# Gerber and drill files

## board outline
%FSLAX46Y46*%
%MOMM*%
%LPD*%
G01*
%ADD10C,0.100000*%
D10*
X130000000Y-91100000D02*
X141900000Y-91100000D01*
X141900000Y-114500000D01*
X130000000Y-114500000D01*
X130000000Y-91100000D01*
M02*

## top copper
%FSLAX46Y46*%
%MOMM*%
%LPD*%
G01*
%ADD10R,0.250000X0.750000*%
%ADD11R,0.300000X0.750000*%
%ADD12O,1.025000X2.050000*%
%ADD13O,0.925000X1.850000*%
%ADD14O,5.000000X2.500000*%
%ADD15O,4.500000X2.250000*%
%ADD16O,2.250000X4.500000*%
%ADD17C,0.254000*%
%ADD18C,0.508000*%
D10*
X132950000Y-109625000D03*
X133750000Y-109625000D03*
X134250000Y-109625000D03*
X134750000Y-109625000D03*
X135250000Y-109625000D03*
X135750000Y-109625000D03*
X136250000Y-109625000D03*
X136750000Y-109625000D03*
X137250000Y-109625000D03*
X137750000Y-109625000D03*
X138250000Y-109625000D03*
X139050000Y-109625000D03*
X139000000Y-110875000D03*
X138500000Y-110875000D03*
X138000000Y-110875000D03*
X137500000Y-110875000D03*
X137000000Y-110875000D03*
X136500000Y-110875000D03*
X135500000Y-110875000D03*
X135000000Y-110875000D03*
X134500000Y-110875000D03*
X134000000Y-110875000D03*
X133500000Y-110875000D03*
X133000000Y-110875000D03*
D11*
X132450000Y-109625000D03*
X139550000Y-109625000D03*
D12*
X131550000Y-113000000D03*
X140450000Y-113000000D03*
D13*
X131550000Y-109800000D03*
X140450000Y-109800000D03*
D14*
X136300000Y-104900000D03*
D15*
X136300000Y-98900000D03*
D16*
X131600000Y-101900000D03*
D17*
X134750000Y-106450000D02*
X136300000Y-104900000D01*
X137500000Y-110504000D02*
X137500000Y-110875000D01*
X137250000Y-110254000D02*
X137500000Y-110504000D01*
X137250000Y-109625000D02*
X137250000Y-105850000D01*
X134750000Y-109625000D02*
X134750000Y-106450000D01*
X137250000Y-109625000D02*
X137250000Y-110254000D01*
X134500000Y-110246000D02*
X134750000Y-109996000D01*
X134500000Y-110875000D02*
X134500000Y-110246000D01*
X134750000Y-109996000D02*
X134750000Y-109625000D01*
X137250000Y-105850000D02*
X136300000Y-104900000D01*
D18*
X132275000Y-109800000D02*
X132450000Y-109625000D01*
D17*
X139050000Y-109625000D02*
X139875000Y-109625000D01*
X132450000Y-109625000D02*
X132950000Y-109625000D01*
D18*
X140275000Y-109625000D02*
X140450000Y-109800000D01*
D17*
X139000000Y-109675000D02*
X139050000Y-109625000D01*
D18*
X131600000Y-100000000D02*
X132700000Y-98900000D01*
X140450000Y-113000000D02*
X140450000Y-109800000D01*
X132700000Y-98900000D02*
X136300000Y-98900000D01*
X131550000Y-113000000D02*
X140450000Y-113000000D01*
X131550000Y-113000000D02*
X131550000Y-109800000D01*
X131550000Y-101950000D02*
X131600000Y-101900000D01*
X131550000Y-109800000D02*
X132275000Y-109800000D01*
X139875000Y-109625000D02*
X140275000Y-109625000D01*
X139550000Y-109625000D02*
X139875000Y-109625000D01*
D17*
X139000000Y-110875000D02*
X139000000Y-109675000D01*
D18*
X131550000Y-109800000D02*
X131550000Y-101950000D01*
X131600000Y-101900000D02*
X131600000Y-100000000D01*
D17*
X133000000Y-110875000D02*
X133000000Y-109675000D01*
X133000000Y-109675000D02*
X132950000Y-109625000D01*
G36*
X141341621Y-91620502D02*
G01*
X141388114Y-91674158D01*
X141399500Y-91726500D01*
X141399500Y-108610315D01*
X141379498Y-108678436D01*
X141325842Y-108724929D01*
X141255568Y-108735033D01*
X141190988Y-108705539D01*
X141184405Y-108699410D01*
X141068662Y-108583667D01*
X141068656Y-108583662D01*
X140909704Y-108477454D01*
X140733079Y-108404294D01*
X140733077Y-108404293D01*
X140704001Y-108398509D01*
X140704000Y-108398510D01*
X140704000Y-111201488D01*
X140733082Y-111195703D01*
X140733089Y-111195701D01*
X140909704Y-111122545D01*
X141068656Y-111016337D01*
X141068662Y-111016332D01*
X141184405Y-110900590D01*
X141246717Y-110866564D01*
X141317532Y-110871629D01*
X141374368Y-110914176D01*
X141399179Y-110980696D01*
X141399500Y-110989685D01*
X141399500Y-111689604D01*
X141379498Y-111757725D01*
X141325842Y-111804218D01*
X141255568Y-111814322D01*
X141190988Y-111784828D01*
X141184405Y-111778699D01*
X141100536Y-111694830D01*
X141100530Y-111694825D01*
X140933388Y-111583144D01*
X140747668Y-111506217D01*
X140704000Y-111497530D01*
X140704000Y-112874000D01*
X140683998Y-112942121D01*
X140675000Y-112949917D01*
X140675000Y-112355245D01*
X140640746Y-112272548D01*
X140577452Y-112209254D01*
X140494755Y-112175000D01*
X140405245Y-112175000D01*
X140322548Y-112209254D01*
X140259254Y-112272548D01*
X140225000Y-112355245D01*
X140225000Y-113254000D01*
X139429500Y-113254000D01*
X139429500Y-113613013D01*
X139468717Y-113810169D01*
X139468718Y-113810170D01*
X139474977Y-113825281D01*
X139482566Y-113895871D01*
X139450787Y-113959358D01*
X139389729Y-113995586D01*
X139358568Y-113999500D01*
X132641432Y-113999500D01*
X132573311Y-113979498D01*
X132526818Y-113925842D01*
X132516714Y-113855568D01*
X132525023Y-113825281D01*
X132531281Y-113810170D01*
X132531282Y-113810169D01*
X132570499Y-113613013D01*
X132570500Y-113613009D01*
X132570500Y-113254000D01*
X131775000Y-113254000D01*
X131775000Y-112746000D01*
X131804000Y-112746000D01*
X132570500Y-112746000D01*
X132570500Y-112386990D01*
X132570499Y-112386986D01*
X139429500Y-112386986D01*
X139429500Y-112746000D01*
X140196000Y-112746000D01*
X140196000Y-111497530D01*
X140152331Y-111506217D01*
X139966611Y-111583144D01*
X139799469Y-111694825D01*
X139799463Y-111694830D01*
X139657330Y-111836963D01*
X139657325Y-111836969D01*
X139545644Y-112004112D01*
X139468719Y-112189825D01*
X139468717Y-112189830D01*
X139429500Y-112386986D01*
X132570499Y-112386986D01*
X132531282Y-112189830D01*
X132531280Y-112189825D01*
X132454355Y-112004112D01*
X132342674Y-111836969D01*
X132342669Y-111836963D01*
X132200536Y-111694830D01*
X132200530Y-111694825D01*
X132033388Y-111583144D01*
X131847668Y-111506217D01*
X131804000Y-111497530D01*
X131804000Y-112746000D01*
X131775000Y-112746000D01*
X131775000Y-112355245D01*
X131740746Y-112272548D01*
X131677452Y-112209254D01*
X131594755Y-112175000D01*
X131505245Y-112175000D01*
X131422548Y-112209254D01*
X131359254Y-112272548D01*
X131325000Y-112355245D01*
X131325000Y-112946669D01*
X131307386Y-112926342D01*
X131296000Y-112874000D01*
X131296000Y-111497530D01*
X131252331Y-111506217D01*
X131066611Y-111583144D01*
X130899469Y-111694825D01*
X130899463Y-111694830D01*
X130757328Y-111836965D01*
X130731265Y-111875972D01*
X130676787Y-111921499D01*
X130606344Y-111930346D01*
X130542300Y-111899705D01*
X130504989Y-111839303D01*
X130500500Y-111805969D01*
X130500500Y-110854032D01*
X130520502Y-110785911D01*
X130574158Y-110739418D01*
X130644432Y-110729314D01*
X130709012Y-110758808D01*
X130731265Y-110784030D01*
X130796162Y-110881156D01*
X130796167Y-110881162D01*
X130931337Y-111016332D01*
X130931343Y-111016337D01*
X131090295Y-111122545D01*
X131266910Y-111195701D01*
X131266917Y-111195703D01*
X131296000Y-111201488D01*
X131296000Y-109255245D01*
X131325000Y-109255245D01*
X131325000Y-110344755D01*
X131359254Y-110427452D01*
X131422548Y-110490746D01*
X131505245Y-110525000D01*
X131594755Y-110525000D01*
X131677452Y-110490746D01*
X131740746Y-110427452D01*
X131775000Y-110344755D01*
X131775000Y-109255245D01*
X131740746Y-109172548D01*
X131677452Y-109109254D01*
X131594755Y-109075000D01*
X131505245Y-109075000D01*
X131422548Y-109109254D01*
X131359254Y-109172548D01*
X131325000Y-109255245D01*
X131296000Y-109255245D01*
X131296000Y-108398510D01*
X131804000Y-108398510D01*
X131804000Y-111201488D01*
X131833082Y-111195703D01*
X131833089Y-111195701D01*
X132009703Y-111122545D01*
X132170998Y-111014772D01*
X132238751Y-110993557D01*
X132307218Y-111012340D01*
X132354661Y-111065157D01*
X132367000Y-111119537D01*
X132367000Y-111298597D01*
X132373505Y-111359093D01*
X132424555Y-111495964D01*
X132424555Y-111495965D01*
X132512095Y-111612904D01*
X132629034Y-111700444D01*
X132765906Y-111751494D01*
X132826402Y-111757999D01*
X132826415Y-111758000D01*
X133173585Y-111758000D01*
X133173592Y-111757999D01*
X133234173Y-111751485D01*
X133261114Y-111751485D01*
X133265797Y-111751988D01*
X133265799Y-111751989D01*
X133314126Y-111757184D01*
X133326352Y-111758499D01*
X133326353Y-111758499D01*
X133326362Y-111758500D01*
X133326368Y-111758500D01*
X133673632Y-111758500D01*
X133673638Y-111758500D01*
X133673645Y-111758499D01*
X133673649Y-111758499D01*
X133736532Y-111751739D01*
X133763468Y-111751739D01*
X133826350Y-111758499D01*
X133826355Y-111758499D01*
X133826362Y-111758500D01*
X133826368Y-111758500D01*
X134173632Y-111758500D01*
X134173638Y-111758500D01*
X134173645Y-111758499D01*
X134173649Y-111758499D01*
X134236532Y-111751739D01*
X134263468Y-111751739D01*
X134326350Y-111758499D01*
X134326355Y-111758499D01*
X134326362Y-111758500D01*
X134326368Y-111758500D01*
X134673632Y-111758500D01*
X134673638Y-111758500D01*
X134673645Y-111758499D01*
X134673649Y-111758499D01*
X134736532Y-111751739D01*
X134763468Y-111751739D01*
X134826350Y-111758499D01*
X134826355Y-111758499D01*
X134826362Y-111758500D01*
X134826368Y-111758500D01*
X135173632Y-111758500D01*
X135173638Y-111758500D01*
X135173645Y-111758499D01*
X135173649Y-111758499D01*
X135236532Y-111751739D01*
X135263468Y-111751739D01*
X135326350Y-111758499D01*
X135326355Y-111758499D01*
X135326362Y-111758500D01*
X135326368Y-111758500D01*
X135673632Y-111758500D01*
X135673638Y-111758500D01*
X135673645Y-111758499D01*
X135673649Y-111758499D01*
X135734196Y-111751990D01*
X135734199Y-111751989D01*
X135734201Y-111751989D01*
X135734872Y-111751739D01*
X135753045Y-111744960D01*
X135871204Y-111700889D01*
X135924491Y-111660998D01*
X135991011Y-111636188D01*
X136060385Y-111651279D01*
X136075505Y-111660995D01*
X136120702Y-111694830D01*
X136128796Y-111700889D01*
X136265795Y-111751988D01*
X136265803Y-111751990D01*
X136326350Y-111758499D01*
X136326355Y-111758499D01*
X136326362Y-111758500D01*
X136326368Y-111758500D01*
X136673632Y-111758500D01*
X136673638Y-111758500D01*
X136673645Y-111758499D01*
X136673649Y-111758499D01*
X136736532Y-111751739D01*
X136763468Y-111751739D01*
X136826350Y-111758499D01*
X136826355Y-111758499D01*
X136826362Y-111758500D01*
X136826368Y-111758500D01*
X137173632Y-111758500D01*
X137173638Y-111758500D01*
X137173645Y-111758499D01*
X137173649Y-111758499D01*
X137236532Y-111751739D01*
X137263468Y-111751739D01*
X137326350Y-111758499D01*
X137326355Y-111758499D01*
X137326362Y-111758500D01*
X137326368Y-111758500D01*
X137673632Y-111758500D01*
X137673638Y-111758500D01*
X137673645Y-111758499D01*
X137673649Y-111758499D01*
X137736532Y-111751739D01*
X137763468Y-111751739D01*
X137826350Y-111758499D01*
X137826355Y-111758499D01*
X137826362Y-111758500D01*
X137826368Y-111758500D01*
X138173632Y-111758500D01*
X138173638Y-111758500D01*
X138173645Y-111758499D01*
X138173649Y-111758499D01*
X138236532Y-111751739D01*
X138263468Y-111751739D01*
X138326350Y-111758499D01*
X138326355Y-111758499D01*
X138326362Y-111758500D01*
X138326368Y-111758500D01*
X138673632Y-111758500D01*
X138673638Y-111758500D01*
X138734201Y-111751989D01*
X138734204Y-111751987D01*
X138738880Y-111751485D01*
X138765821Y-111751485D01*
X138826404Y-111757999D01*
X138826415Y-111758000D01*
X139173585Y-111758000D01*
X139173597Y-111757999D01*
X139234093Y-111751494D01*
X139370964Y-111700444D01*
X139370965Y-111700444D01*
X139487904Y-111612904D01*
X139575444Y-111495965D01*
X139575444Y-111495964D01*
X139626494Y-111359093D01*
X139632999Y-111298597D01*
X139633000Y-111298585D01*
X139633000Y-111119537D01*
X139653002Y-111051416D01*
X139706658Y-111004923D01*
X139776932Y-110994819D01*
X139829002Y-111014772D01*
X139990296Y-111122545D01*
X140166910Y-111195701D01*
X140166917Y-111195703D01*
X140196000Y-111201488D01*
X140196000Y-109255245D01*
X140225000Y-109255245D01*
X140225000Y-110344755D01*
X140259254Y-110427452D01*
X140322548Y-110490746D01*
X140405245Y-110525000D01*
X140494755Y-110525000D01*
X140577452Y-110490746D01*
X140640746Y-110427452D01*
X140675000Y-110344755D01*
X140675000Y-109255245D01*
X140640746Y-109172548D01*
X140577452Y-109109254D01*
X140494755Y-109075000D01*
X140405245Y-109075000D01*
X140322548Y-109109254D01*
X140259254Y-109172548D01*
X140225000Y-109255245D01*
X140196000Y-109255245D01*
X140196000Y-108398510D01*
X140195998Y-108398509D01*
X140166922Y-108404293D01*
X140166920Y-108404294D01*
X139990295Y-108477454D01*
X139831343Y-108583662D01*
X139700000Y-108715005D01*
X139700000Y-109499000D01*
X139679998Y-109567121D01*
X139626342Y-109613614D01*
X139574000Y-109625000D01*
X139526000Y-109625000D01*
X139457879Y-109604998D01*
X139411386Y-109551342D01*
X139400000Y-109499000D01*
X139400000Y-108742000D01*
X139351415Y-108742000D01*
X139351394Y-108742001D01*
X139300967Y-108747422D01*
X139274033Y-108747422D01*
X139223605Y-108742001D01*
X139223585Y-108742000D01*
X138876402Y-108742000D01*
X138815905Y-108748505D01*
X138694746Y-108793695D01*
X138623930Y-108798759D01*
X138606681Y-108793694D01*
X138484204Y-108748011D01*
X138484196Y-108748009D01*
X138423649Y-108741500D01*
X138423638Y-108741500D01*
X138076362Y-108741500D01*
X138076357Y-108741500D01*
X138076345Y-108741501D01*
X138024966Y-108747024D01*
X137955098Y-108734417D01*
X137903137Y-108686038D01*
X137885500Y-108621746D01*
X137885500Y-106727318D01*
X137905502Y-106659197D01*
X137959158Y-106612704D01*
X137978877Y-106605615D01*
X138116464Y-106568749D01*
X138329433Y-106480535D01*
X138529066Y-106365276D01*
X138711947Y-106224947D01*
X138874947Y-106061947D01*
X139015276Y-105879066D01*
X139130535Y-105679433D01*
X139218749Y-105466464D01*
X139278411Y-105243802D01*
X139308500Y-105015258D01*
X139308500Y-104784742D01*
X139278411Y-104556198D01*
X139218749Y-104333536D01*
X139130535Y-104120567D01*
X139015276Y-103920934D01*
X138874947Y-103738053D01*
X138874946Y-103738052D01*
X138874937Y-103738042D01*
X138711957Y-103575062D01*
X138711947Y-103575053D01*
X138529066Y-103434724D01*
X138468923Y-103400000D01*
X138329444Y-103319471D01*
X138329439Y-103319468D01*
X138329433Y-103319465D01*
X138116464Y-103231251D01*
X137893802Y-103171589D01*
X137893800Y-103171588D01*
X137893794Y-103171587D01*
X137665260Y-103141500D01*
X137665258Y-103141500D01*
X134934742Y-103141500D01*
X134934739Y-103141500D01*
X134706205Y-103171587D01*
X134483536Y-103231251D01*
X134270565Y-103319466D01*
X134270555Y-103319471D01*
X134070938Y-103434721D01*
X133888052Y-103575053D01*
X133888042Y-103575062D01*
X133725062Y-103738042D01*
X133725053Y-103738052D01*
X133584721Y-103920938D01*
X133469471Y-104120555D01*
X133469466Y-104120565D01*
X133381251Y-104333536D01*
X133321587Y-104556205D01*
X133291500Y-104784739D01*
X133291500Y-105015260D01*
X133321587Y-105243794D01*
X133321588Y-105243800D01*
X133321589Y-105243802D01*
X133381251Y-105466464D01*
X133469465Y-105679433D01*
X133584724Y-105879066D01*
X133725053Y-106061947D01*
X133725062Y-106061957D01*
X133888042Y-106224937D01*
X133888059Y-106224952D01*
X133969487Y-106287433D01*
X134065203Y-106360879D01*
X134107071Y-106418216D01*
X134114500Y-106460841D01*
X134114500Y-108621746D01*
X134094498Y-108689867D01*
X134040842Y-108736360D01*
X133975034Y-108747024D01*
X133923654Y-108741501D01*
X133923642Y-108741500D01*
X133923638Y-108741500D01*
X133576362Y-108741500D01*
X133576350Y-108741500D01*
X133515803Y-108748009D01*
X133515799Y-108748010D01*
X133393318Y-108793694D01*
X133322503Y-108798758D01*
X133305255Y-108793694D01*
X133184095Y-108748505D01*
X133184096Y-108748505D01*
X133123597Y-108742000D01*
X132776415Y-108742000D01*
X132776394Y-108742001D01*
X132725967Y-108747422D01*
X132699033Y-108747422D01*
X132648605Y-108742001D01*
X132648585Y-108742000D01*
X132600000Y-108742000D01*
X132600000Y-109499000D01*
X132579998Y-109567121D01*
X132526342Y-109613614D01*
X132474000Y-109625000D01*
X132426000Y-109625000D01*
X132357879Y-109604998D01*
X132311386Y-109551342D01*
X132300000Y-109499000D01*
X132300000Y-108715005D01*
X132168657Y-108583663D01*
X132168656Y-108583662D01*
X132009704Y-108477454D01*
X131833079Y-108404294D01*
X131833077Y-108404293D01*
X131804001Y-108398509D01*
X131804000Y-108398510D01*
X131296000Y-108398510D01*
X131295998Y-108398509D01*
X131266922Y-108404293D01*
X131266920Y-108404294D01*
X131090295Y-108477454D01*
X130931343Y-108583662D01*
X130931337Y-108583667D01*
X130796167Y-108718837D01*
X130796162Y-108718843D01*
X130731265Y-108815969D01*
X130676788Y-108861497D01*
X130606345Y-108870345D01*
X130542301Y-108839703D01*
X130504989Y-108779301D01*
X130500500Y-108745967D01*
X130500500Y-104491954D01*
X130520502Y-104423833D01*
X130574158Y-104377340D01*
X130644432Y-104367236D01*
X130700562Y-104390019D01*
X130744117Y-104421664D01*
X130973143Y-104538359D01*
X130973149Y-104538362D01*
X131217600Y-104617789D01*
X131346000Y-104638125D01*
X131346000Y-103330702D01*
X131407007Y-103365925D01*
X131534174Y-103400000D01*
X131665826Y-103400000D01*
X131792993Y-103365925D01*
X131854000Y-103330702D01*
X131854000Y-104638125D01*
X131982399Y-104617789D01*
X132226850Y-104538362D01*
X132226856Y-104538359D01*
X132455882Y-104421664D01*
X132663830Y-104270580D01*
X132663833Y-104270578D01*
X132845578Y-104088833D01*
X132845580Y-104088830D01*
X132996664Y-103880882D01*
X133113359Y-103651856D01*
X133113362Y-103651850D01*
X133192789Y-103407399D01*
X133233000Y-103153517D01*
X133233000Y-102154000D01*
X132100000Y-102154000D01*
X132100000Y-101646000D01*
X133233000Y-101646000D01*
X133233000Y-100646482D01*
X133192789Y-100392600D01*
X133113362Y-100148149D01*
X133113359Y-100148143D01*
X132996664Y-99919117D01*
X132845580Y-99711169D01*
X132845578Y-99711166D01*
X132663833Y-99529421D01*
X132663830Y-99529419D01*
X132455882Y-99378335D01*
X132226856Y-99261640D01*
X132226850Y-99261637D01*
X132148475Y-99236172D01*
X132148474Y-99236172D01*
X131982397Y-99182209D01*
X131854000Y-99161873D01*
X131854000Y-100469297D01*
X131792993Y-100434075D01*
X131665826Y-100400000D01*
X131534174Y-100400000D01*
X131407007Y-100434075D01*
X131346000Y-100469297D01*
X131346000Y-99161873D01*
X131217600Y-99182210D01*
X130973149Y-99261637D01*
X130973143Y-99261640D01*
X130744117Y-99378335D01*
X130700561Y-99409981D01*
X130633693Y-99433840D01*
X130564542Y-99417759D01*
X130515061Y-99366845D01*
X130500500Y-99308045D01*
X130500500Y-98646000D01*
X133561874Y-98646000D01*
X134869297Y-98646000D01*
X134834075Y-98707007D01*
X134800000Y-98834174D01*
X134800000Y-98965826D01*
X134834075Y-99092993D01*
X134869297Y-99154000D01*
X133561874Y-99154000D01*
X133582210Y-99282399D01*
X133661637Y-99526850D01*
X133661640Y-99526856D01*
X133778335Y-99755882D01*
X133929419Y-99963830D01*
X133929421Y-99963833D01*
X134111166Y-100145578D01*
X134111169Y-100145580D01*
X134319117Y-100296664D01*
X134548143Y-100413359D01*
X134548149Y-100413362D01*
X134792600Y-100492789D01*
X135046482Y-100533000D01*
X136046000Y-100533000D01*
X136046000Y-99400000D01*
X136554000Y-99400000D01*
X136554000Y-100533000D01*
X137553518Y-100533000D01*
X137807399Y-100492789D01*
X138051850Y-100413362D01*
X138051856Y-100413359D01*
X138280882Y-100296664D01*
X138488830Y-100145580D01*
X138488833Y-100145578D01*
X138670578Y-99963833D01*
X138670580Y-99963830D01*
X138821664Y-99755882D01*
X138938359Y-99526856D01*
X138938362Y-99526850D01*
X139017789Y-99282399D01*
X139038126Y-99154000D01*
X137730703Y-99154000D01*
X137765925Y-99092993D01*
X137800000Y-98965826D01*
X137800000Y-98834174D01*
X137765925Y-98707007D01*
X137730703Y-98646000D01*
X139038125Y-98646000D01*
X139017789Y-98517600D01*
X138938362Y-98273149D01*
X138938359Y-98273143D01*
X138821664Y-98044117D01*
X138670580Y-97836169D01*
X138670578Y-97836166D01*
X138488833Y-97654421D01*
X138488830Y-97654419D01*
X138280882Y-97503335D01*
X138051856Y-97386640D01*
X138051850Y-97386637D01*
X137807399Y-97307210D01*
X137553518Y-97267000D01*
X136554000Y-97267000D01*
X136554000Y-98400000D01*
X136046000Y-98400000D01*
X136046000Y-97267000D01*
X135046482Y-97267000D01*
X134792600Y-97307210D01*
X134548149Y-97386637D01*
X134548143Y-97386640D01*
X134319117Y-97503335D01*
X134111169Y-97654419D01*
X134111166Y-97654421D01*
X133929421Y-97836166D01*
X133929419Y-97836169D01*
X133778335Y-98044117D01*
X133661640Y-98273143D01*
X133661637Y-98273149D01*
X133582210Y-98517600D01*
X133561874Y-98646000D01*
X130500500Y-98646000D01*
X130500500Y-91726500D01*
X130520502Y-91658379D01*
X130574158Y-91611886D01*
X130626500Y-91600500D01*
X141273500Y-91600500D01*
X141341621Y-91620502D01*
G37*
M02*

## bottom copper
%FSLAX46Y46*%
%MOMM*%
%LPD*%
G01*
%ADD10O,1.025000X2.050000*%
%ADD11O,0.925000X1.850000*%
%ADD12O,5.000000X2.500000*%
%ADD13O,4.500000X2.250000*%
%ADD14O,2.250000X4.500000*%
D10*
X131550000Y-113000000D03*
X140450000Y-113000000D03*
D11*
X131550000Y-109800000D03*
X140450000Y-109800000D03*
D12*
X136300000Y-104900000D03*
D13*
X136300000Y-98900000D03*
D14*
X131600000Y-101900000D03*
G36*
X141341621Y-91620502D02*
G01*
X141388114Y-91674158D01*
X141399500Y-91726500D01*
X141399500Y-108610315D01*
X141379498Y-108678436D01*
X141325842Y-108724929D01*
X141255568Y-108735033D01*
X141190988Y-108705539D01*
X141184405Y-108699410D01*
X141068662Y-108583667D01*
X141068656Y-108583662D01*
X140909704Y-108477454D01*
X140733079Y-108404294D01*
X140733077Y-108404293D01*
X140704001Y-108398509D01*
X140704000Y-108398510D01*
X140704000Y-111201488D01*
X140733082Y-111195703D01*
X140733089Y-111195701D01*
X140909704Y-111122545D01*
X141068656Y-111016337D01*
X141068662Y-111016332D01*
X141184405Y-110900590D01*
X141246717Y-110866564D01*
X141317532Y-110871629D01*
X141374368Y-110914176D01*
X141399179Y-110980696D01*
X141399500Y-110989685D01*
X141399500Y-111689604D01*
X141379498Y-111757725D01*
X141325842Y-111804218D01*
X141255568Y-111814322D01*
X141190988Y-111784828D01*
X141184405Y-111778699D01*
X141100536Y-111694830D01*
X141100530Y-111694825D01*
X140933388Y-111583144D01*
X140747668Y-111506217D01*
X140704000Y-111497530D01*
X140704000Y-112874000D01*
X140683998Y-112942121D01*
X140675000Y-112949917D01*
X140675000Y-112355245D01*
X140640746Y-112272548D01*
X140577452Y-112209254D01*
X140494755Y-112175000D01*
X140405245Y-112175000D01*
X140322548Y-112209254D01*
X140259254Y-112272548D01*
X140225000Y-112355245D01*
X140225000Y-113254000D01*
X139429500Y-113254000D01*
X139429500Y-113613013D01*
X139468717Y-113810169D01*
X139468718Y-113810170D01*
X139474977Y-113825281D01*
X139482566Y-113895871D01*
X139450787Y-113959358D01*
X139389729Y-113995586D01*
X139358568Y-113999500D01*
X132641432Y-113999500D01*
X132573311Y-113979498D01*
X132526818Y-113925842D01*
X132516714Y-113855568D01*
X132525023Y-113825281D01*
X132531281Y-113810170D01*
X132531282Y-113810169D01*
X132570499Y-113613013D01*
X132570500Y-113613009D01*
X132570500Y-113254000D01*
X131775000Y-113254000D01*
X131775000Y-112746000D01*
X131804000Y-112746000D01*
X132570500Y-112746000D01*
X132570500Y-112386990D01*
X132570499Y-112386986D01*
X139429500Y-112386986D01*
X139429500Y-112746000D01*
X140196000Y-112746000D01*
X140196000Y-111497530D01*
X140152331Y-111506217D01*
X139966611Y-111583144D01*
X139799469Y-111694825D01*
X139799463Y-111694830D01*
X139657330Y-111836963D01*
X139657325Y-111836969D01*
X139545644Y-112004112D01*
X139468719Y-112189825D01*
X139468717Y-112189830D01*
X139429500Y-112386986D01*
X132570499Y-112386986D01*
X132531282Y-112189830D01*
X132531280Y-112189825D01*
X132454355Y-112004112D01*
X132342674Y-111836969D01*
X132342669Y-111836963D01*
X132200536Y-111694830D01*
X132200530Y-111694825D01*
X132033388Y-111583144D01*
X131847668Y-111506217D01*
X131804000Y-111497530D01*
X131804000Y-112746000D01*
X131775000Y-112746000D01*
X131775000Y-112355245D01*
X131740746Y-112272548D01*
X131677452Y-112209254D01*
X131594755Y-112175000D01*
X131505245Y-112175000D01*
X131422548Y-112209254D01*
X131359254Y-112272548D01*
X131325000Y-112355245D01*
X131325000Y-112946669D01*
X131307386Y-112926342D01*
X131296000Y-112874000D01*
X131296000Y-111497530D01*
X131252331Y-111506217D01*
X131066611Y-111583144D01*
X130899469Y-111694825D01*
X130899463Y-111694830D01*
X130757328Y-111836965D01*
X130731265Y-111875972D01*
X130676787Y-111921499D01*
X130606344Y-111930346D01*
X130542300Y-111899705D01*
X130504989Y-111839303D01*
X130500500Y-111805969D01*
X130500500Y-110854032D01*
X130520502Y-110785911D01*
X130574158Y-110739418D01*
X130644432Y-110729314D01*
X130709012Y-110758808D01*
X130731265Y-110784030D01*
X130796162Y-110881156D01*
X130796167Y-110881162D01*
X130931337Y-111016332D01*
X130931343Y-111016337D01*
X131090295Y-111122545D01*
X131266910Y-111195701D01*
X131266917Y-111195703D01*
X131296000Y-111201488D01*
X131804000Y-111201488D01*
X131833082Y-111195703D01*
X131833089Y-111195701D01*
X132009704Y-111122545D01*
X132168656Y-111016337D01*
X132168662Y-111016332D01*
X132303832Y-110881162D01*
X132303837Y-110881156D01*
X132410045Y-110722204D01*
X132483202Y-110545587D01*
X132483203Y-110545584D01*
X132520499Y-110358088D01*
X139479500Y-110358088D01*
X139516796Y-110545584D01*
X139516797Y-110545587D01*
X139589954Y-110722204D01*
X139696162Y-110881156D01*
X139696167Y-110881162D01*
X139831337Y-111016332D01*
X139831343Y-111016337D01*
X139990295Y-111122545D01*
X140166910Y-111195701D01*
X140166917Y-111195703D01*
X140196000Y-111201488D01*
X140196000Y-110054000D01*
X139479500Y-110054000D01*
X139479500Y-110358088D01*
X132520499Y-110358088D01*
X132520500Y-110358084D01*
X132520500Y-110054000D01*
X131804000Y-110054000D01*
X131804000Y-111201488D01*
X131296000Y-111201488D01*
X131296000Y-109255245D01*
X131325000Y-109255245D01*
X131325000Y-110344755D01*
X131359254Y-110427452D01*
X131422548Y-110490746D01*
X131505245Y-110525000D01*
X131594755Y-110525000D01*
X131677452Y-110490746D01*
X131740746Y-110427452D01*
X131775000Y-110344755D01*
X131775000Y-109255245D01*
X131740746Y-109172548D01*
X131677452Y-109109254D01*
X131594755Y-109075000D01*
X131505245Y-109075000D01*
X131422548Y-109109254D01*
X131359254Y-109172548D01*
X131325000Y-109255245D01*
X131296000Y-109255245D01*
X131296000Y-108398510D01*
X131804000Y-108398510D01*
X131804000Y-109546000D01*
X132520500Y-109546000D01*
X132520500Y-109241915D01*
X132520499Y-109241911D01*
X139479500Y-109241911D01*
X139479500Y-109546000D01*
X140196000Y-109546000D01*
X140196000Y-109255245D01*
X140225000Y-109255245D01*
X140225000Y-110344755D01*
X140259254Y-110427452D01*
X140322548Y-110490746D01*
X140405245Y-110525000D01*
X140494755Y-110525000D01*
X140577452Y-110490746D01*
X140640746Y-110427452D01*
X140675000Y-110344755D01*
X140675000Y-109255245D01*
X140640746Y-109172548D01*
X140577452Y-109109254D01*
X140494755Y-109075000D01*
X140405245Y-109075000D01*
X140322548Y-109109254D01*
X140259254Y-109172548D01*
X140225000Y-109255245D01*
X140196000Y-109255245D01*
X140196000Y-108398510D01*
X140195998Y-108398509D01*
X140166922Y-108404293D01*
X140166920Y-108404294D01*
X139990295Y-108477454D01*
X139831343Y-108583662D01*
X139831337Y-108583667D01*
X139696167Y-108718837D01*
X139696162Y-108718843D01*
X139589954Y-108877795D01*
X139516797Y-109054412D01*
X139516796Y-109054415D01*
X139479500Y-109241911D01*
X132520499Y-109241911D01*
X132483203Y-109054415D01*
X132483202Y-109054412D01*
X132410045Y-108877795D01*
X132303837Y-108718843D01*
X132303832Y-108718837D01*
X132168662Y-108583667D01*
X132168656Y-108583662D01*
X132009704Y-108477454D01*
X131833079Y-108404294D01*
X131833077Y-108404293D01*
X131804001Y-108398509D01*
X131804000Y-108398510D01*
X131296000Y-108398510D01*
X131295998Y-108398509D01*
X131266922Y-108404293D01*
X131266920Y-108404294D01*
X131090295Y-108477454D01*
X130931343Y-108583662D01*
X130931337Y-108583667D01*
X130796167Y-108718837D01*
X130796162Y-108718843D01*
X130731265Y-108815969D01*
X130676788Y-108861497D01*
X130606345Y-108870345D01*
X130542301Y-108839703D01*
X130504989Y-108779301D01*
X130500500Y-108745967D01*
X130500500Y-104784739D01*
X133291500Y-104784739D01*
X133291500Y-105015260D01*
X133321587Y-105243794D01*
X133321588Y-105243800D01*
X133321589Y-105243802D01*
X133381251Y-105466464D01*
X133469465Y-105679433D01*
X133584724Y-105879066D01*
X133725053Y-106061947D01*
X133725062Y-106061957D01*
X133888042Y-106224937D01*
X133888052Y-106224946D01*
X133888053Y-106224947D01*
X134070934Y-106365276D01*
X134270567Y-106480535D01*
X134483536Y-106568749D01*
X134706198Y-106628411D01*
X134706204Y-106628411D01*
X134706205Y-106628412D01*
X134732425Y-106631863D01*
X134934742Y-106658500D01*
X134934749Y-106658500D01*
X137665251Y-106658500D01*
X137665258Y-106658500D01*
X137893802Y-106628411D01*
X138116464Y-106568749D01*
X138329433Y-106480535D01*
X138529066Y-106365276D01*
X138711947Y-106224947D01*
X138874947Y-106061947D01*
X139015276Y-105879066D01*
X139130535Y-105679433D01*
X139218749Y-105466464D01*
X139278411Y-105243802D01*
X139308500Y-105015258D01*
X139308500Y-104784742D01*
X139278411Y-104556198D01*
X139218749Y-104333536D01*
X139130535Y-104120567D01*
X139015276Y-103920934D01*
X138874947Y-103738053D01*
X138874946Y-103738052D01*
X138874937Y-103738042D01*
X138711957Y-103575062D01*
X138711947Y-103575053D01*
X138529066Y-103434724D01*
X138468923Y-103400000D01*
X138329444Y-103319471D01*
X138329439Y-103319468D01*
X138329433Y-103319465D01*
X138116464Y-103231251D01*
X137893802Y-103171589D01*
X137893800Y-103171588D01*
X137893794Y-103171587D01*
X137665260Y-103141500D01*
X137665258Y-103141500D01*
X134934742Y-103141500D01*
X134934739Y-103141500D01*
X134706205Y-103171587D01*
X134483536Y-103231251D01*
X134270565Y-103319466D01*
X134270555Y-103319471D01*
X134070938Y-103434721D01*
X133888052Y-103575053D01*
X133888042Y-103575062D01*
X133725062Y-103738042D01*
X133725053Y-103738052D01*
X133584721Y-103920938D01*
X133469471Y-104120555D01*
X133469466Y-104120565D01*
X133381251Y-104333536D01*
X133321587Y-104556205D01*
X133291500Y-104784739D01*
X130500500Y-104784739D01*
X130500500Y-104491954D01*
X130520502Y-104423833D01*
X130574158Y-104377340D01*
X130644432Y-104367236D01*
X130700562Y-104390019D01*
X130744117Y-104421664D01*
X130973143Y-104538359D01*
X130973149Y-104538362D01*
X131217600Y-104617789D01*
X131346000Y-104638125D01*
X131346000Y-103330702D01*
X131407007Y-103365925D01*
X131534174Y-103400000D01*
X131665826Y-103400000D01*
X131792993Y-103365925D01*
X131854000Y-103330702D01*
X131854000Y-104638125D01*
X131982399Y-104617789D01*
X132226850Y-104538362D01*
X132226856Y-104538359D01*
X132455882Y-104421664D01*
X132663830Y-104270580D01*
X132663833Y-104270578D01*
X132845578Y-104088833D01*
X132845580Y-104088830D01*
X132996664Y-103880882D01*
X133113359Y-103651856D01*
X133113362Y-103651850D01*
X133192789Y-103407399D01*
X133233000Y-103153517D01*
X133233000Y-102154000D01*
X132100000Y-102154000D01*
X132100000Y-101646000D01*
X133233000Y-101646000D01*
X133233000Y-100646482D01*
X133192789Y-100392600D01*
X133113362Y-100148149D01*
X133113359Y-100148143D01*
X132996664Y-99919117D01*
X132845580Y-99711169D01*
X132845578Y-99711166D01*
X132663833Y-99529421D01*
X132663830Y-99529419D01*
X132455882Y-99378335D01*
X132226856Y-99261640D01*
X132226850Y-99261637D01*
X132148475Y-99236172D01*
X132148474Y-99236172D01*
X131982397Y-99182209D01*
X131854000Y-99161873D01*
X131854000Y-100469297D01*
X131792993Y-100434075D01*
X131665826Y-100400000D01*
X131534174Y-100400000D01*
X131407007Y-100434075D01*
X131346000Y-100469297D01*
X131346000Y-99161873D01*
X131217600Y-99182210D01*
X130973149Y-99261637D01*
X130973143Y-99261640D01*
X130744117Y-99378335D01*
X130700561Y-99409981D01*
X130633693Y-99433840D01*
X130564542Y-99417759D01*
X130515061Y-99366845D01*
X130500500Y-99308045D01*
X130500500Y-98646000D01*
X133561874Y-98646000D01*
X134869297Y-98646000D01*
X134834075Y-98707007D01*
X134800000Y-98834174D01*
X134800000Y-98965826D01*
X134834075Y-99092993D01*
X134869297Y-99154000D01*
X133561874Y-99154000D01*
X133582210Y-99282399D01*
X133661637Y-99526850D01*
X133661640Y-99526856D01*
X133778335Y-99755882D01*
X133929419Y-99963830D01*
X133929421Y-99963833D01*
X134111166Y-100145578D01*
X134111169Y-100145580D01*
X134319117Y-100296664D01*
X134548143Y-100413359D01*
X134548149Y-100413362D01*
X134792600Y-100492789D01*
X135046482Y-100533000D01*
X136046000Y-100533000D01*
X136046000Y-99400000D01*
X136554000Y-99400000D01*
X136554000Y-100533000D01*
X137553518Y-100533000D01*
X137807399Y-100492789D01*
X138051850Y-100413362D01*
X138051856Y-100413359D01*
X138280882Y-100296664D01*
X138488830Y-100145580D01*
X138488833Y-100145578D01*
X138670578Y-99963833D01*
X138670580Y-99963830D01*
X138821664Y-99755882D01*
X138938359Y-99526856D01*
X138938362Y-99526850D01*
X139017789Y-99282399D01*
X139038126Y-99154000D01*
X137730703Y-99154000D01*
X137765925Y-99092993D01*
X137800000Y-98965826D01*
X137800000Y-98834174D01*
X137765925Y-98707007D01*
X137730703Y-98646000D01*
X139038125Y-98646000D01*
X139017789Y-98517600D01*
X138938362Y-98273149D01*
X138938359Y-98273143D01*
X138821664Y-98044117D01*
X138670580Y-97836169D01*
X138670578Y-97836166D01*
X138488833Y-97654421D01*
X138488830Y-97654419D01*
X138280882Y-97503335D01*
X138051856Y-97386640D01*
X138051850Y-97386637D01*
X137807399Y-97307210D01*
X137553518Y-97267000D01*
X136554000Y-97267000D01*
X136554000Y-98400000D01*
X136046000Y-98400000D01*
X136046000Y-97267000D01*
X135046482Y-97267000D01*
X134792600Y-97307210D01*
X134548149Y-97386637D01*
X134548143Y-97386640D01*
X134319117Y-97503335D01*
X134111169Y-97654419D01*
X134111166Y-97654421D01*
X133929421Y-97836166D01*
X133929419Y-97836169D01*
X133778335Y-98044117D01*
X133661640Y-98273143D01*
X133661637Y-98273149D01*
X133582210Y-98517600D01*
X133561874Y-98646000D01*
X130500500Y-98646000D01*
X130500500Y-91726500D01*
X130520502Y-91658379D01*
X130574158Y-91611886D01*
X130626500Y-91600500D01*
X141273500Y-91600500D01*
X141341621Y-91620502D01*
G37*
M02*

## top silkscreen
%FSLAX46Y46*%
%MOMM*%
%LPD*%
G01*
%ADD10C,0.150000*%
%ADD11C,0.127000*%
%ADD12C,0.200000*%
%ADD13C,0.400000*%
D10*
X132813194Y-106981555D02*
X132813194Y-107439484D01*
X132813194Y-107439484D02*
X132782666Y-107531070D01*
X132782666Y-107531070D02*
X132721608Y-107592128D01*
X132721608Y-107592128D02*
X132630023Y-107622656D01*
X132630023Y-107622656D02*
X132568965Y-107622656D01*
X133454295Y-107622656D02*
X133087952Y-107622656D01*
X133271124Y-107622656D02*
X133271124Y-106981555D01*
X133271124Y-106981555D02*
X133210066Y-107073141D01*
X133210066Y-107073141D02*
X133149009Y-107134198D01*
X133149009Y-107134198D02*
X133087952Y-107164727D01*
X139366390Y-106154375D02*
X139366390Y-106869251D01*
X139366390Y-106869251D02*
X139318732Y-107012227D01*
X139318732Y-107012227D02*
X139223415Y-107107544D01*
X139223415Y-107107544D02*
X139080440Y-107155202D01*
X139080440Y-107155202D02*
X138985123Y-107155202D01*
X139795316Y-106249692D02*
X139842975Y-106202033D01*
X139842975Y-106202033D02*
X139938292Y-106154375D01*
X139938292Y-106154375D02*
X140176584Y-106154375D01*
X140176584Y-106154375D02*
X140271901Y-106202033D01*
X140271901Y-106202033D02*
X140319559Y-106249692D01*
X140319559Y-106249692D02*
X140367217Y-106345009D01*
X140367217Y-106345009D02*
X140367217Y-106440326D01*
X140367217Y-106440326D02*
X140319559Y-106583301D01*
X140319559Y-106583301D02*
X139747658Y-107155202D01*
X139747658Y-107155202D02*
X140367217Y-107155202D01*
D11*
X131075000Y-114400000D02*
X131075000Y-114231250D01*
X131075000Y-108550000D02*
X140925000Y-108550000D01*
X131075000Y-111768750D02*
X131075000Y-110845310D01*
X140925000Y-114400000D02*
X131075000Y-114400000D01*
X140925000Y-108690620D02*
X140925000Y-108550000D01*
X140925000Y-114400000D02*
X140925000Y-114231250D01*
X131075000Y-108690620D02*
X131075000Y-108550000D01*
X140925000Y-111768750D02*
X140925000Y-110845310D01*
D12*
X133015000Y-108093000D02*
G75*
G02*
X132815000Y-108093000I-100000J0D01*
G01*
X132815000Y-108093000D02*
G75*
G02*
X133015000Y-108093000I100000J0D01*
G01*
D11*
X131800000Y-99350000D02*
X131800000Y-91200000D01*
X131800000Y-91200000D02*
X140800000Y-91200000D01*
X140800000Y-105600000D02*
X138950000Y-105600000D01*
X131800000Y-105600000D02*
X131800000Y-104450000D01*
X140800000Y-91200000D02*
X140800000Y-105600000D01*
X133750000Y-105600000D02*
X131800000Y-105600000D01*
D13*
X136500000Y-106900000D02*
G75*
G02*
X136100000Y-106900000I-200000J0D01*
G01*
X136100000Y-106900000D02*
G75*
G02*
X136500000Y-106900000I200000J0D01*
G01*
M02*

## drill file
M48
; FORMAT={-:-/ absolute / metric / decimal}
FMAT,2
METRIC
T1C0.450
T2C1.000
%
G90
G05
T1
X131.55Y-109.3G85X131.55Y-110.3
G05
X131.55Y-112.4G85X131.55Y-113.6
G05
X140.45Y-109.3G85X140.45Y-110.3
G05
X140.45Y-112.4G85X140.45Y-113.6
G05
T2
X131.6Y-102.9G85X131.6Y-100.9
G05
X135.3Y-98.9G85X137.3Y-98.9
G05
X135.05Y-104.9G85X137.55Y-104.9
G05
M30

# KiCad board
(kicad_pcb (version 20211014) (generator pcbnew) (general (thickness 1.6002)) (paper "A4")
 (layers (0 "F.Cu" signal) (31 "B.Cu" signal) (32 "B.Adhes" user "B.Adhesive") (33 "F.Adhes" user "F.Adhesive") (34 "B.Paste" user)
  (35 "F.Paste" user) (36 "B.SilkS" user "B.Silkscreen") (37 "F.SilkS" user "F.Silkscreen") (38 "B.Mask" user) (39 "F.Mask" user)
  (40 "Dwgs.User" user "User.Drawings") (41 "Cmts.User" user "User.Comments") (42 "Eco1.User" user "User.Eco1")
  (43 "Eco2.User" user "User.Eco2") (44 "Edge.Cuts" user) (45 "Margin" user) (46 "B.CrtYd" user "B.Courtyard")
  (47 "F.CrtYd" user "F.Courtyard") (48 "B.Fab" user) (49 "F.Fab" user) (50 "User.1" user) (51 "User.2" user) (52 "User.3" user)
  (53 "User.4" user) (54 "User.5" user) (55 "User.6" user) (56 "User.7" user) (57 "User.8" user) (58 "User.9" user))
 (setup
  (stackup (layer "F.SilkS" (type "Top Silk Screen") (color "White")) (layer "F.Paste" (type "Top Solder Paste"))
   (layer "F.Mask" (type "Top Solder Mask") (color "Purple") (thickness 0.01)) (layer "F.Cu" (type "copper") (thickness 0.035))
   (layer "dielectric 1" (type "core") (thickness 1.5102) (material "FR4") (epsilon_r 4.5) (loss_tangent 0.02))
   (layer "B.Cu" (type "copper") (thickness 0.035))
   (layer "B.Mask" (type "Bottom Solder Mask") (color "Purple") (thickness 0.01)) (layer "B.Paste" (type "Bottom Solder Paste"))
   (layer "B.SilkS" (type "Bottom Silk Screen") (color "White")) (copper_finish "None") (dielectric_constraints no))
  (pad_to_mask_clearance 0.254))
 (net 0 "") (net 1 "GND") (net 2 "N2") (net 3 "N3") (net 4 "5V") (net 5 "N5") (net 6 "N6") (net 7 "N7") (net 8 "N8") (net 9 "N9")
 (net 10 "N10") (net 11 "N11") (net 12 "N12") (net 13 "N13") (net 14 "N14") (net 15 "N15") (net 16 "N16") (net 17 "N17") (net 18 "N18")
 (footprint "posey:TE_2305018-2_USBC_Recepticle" (layer "F.Cu") (at 136 113)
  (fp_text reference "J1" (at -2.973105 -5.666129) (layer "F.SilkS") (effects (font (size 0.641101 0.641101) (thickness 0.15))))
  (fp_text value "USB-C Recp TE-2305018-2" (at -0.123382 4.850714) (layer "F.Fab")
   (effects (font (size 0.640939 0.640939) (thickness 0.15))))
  (fp_line (start -4.925 1.4) (end -4.925 1.23125) (layer "F.SilkS") (width 0.127))
  (fp_line (start -4.925 -4.45) (end 4.925 -4.45) (layer "F.SilkS") (width 0.127))
  (fp_line (start -4.925 -1.23125) (end -4.925 -2.15469) (layer "F.SilkS") (width 0.127))
  (fp_line (start 4.925 1.4) (end -4.925 1.4) (layer "F.SilkS") (width 0.127))
  (fp_line (start 4.925 -4.30938) (end 4.925 -4.45) (layer "F.SilkS") (width 0.127))
  (fp_line (start 4.925 1.4) (end 4.925 1.23125) (layer "F.SilkS") (width 0.127))
  (fp_line (start -4.925 -4.30938) (end -4.925 -4.45) (layer "F.SilkS") (width 0.127))
  (fp_line (start 4.925 -1.23125) (end 4.925 -2.15469) (layer "F.SilkS") (width 0.127))
  (fp_circle (center -3.085 -4.907) (end -2.985 -4.907) (layer "F.SilkS") (width 0.2) (fill none))
  (pad "A1" smd rect (at -3.05 -3.375) (size 0.25 0.75) (layers "F.Cu" "F.Paste" "F.Mask") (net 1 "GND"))
  (pad "A2" smd rect (at -2.25 -3.375) (size 0.25 0.75) (layers "F.Cu" "F.Paste" "F.Mask") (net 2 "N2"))
  (pad "A3" smd rect (at -1.75 -3.375) (size 0.25 0.75) (layers "F.Cu" "F.Paste" "F.Mask") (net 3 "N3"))
  (pad "A4" smd rect (at -1.25 -3.375) (size 0.25 0.75) (layers "F.Cu" "F.Paste" "F.Mask") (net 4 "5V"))
  (pad "A5" smd rect (at -0.75 -3.375) (size 0.25 0.75) (layers "F.Cu" "F.Paste" "F.Mask") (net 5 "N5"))
  (pad "A6" smd rect (at -0.25 -3.375) (size 0.25 0.75) (layers "F.Cu" "F.Paste" "F.Mask") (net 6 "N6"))
  (pad "A7" smd rect (at 0.25 -3.375) (size 0.25 0.75) (layers "F.Cu" "F.Paste" "F.Mask") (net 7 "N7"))
  (pad "A8" smd rect (at 0.75 -3.375) (size 0.25 0.75) (layers "F.Cu" "F.Paste" "F.Mask") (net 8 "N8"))
  (pad "A9" smd rect (at 1.25 -3.375) (size 0.25 0.75) (layers "F.Cu" "F.Paste" "F.Mask") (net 4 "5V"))
  (pad "A10" smd rect (at 1.75 -3.375) (size 0.25 0.75) (layers "F.Cu" "F.Paste" "F.Mask") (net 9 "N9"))
  (pad "A11" smd rect (at 2.25 -3.375) (size 0.25 0.75) (layers "F.Cu" "F.Paste" "F.Mask") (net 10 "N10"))
  (pad "A12" smd rect (at 3.05 -3.375) (size 0.25 0.75) (layers "F.Cu" "F.Paste" "F.Mask") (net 1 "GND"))
  (pad "B1" smd rect (at 3 -2.125) (size 0.25 0.75) (layers "F.Cu" "F.Paste" "F.Mask") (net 1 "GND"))
  (pad "B2" smd rect (at 2.5 -2.125) (size 0.25 0.75) (layers "F.Cu" "F.Paste" "F.Mask") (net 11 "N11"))
  (pad "B3" smd rect (at 2 -2.125) (size 0.25 0.75) (layers "F.Cu" "F.Paste" "F.Mask") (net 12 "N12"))
  (pad "B4" smd rect (at 1.5 -2.125) (size 0.25 0.75) (layers "F.Cu" "F.Paste" "F.Mask") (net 4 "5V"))
  (pad "B5" smd rect (at 1 -2.125) (size 0.25 0.75) (layers "F.Cu" "F.Paste" "F.Mask") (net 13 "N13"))
  (pad "B6" smd rect (at 0.5 -2.125) (size 0.25 0.75) (layers "F.Cu" "F.Paste" "F.Mask") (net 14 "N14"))
  (pad "B7" smd rect (at -0.5 -2.125) (size 0.25 0.75) (layers "F.Cu" "F.Paste" "F.Mask") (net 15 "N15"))
  (pad "B8" smd rect (at -1 -2.125) (size 0.25 0.75) (layers "F.Cu" "F.Paste" "F.Mask") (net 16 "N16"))
  (pad "B9" smd rect (at -1.5 -2.125) (size 0.25 0.75) (layers "F.Cu" "F.Paste" "F.Mask") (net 4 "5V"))
  (pad "B10" smd rect (at -2 -2.125) (size 0.25 0.75) (layers "F.Cu" "F.Paste" "F.Mask") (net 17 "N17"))
  (pad "B11" smd rect (at -2.5 -2.125) (size 0.25 0.75) (layers "F.Cu" "F.Paste" "F.Mask") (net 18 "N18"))
  (pad "B12" smd rect (at -3 -2.125) (size 0.25 0.75) (layers "F.Cu" "F.Paste" "F.Mask") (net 1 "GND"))
  (pad "G1" smd rect (at -3.55 -3.375) (size 0.3 0.75) (layers "F.Cu" "F.Paste" "F.Mask") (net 1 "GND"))
  (pad "G2" smd rect (at 3.55 -3.375) (size 0.3 0.75) (layers "F.Cu" "F.Paste" "F.Mask") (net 1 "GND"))
  (pad "S1" thru_hole oval (at -4.45 0) (size 1.025 2.05) (drill oval 0.45 1.65) (layers *.Cu *.Mask) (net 1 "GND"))
  (pad "S2" thru_hole oval (at 4.45 0) (size 1.025 2.05) (drill oval 0.45 1.65) (layers *.Cu *.Mask) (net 1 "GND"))
  (pad "S3" thru_hole oval (at -4.45 -3.2) (size 0.925 1.85) (drill oval 0.45 1.45) (layers *.Cu *.Mask) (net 1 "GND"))
  (pad "S4" thru_hole oval (at 4.45 -3.2) (size 0.925 1.85) (drill oval 0.45 1.45) (layers *.Cu *.Mask) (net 1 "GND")))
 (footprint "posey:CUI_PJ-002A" (layer "F.Cu") (at 136.3 104.9 90)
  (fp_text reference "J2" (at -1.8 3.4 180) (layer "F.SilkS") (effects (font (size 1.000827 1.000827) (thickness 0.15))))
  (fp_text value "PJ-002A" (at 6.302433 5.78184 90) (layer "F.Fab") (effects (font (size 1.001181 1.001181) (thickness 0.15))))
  (fp_line (start 5.55 -4.5) (end 13.7 -4.5) (layer "F.SilkS") (width 0.127))
  (fp_line (start 13.7 -4.5) (end 13.7 4.5) (layer "F.SilkS") (width 0.127))
  (fp_line (start -0.7 4.5) (end -0.7 2.65) (layer "F.SilkS") (width 0.127))
  (fp_line (start -0.7 -4.5) (end 0.45 -4.5) (layer "F.SilkS") (width 0.127))
  (fp_line (start 13.7 4.5) (end -0.7 4.5) (layer "F.SilkS") (width 0.127))
  (fp_line (start -0.7 -2.55) (end -0.7 -4.5) (layer "F.SilkS") (width 0.127))
  (fp_circle (center -2 0) (end -1.8 0) (layer "F.SilkS") (width 0.4) (fill none))
  (pad "1" thru_hole oval (at 0 0 90) (size 2.5 5) (drill oval 1 3.5) (layers *.Cu *.Mask) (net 4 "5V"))
  (pad "2" thru_hole oval (at 6 0 90) (size 2.25 4.5) (drill oval 1 3) (layers *.Cu *.Mask) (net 1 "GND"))
  (pad "3" thru_hole oval (at 3 -4.7 90) (size 4.5 2.25) (drill oval 3 1) (layers *.Cu *.Mask) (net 1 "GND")))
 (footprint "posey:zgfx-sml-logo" (layer "B.Cu") (at 137.8 92.9 180)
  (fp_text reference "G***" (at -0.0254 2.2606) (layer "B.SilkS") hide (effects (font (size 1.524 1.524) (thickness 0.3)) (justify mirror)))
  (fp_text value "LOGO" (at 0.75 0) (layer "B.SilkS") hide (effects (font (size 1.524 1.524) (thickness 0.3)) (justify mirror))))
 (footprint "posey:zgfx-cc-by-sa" (layer "B.Cu") (at 132.9 96.1 180)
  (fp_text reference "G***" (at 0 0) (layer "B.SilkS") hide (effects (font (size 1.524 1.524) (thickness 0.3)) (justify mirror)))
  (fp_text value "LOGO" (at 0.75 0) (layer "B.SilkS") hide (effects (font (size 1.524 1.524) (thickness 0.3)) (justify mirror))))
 (gr_rect (start 130 91.1) (end 141.9 114.5) (layer "Edge.Cuts") (width 0.1) (fill none))
 (segment (start 134.75 106.45) (end 136.3 104.9) (width 0.254) (layer "F.Cu") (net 4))
 (segment (start 137.5 110.504) (end 137.5 110.875) (width 0.254) (layer "F.Cu") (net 4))
 (segment (start 137.25 110.254) (end 137.5 110.504) (width 0.254) (layer "F.Cu") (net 4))
 (segment (start 137.25 109.625) (end 137.25 105.85) (width 0.254) (layer "F.Cu") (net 4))
 (segment (start 134.75 109.625) (end 134.75 106.45) (width 0.254) (layer "F.Cu") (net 4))
 (segment (start 137.25 109.625) (end 137.25 110.254) (width 0.254) (layer "F.Cu") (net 4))
 (segment (start 134.5 110.246) (end 134.75 109.996) (width 0.254) (layer "F.Cu") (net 4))
 (segment (start 134.5 110.875) (end 134.5 110.246) (width 0.254) (layer "F.Cu") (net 4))
 (segment (start 134.75 109.996) (end 134.75 109.625) (width 0.254) (layer "F.Cu") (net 4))
 (segment (start 137.25 105.85) (end 136.3 104.9) (width 0.254) (layer "F.Cu") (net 4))
 (segment (start 132.275 109.8) (end 132.45 109.625) (width 0.508) (layer "F.Cu") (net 1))
 (segment (start 139.05 109.625) (end 139.875 109.625) (width 0.254) (layer "F.Cu") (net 1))
 (segment (start 132.45 109.625) (end 132.95 109.625) (width 0.254) (layer "F.Cu") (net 1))
 (segment (start 140.275 109.625) (end 140.45 109.8) (width 0.508) (layer "F.Cu") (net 1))
 (segment (start 139 109.675) (end 139.05 109.625) (width 0.254) (layer "F.Cu") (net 1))
 (segment (start 131.6 100) (end 132.7 98.9) (width 0.508) (layer "F.Cu") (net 1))
 (segment (start 140.45 113) (end 140.45 109.8) (width 0.508) (layer "F.Cu") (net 1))
 (segment (start 132.7 98.9) (end 136.3 98.9) (width 0.508) (layer "F.Cu") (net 1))
 (segment (start 131.55 113) (end 140.45 113) (width 0.508) (layer "F.Cu") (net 1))
 (segment (start 131.55 113) (end 131.55 109.8) (width 0.508) (layer "F.Cu") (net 1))
 (segment (start 131.55 101.95) (end 131.6 101.9) (width 0.508) (layer "F.Cu") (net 1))
 (segment (start 131.55 109.8) (end 132.275 109.8) (width 0.508) (layer "F.Cu") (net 1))
 (segment (start 139.875 109.625) (end 140.275 109.625) (width 0.508) (layer "F.Cu") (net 1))
 (segment (start 139.55 109.625) (end 139.875 109.625) (width 0.508) (layer "F.Cu") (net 1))
 (segment (start 139 110.875) (end 139 109.675) (width 0.254) (layer "F.Cu") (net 1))
 (segment (start 131.55 109.8) (end 131.55 101.95) (width 0.508) (layer "F.Cu") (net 1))
 (segment (start 131.6 101.9) (end 131.6 100) (width 0.508) (layer "F.Cu") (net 1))
 (segment (start 133 110.875) (end 133 109.675) (width 0.254) (layer "F.Cu") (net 1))
 (segment (start 133 109.675) (end 132.95 109.625) (width 0.254) (layer "F.Cu") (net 1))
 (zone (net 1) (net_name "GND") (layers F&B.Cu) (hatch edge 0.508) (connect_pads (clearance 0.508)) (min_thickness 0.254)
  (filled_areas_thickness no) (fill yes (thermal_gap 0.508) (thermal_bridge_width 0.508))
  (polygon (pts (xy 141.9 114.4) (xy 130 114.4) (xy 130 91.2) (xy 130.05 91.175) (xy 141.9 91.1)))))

